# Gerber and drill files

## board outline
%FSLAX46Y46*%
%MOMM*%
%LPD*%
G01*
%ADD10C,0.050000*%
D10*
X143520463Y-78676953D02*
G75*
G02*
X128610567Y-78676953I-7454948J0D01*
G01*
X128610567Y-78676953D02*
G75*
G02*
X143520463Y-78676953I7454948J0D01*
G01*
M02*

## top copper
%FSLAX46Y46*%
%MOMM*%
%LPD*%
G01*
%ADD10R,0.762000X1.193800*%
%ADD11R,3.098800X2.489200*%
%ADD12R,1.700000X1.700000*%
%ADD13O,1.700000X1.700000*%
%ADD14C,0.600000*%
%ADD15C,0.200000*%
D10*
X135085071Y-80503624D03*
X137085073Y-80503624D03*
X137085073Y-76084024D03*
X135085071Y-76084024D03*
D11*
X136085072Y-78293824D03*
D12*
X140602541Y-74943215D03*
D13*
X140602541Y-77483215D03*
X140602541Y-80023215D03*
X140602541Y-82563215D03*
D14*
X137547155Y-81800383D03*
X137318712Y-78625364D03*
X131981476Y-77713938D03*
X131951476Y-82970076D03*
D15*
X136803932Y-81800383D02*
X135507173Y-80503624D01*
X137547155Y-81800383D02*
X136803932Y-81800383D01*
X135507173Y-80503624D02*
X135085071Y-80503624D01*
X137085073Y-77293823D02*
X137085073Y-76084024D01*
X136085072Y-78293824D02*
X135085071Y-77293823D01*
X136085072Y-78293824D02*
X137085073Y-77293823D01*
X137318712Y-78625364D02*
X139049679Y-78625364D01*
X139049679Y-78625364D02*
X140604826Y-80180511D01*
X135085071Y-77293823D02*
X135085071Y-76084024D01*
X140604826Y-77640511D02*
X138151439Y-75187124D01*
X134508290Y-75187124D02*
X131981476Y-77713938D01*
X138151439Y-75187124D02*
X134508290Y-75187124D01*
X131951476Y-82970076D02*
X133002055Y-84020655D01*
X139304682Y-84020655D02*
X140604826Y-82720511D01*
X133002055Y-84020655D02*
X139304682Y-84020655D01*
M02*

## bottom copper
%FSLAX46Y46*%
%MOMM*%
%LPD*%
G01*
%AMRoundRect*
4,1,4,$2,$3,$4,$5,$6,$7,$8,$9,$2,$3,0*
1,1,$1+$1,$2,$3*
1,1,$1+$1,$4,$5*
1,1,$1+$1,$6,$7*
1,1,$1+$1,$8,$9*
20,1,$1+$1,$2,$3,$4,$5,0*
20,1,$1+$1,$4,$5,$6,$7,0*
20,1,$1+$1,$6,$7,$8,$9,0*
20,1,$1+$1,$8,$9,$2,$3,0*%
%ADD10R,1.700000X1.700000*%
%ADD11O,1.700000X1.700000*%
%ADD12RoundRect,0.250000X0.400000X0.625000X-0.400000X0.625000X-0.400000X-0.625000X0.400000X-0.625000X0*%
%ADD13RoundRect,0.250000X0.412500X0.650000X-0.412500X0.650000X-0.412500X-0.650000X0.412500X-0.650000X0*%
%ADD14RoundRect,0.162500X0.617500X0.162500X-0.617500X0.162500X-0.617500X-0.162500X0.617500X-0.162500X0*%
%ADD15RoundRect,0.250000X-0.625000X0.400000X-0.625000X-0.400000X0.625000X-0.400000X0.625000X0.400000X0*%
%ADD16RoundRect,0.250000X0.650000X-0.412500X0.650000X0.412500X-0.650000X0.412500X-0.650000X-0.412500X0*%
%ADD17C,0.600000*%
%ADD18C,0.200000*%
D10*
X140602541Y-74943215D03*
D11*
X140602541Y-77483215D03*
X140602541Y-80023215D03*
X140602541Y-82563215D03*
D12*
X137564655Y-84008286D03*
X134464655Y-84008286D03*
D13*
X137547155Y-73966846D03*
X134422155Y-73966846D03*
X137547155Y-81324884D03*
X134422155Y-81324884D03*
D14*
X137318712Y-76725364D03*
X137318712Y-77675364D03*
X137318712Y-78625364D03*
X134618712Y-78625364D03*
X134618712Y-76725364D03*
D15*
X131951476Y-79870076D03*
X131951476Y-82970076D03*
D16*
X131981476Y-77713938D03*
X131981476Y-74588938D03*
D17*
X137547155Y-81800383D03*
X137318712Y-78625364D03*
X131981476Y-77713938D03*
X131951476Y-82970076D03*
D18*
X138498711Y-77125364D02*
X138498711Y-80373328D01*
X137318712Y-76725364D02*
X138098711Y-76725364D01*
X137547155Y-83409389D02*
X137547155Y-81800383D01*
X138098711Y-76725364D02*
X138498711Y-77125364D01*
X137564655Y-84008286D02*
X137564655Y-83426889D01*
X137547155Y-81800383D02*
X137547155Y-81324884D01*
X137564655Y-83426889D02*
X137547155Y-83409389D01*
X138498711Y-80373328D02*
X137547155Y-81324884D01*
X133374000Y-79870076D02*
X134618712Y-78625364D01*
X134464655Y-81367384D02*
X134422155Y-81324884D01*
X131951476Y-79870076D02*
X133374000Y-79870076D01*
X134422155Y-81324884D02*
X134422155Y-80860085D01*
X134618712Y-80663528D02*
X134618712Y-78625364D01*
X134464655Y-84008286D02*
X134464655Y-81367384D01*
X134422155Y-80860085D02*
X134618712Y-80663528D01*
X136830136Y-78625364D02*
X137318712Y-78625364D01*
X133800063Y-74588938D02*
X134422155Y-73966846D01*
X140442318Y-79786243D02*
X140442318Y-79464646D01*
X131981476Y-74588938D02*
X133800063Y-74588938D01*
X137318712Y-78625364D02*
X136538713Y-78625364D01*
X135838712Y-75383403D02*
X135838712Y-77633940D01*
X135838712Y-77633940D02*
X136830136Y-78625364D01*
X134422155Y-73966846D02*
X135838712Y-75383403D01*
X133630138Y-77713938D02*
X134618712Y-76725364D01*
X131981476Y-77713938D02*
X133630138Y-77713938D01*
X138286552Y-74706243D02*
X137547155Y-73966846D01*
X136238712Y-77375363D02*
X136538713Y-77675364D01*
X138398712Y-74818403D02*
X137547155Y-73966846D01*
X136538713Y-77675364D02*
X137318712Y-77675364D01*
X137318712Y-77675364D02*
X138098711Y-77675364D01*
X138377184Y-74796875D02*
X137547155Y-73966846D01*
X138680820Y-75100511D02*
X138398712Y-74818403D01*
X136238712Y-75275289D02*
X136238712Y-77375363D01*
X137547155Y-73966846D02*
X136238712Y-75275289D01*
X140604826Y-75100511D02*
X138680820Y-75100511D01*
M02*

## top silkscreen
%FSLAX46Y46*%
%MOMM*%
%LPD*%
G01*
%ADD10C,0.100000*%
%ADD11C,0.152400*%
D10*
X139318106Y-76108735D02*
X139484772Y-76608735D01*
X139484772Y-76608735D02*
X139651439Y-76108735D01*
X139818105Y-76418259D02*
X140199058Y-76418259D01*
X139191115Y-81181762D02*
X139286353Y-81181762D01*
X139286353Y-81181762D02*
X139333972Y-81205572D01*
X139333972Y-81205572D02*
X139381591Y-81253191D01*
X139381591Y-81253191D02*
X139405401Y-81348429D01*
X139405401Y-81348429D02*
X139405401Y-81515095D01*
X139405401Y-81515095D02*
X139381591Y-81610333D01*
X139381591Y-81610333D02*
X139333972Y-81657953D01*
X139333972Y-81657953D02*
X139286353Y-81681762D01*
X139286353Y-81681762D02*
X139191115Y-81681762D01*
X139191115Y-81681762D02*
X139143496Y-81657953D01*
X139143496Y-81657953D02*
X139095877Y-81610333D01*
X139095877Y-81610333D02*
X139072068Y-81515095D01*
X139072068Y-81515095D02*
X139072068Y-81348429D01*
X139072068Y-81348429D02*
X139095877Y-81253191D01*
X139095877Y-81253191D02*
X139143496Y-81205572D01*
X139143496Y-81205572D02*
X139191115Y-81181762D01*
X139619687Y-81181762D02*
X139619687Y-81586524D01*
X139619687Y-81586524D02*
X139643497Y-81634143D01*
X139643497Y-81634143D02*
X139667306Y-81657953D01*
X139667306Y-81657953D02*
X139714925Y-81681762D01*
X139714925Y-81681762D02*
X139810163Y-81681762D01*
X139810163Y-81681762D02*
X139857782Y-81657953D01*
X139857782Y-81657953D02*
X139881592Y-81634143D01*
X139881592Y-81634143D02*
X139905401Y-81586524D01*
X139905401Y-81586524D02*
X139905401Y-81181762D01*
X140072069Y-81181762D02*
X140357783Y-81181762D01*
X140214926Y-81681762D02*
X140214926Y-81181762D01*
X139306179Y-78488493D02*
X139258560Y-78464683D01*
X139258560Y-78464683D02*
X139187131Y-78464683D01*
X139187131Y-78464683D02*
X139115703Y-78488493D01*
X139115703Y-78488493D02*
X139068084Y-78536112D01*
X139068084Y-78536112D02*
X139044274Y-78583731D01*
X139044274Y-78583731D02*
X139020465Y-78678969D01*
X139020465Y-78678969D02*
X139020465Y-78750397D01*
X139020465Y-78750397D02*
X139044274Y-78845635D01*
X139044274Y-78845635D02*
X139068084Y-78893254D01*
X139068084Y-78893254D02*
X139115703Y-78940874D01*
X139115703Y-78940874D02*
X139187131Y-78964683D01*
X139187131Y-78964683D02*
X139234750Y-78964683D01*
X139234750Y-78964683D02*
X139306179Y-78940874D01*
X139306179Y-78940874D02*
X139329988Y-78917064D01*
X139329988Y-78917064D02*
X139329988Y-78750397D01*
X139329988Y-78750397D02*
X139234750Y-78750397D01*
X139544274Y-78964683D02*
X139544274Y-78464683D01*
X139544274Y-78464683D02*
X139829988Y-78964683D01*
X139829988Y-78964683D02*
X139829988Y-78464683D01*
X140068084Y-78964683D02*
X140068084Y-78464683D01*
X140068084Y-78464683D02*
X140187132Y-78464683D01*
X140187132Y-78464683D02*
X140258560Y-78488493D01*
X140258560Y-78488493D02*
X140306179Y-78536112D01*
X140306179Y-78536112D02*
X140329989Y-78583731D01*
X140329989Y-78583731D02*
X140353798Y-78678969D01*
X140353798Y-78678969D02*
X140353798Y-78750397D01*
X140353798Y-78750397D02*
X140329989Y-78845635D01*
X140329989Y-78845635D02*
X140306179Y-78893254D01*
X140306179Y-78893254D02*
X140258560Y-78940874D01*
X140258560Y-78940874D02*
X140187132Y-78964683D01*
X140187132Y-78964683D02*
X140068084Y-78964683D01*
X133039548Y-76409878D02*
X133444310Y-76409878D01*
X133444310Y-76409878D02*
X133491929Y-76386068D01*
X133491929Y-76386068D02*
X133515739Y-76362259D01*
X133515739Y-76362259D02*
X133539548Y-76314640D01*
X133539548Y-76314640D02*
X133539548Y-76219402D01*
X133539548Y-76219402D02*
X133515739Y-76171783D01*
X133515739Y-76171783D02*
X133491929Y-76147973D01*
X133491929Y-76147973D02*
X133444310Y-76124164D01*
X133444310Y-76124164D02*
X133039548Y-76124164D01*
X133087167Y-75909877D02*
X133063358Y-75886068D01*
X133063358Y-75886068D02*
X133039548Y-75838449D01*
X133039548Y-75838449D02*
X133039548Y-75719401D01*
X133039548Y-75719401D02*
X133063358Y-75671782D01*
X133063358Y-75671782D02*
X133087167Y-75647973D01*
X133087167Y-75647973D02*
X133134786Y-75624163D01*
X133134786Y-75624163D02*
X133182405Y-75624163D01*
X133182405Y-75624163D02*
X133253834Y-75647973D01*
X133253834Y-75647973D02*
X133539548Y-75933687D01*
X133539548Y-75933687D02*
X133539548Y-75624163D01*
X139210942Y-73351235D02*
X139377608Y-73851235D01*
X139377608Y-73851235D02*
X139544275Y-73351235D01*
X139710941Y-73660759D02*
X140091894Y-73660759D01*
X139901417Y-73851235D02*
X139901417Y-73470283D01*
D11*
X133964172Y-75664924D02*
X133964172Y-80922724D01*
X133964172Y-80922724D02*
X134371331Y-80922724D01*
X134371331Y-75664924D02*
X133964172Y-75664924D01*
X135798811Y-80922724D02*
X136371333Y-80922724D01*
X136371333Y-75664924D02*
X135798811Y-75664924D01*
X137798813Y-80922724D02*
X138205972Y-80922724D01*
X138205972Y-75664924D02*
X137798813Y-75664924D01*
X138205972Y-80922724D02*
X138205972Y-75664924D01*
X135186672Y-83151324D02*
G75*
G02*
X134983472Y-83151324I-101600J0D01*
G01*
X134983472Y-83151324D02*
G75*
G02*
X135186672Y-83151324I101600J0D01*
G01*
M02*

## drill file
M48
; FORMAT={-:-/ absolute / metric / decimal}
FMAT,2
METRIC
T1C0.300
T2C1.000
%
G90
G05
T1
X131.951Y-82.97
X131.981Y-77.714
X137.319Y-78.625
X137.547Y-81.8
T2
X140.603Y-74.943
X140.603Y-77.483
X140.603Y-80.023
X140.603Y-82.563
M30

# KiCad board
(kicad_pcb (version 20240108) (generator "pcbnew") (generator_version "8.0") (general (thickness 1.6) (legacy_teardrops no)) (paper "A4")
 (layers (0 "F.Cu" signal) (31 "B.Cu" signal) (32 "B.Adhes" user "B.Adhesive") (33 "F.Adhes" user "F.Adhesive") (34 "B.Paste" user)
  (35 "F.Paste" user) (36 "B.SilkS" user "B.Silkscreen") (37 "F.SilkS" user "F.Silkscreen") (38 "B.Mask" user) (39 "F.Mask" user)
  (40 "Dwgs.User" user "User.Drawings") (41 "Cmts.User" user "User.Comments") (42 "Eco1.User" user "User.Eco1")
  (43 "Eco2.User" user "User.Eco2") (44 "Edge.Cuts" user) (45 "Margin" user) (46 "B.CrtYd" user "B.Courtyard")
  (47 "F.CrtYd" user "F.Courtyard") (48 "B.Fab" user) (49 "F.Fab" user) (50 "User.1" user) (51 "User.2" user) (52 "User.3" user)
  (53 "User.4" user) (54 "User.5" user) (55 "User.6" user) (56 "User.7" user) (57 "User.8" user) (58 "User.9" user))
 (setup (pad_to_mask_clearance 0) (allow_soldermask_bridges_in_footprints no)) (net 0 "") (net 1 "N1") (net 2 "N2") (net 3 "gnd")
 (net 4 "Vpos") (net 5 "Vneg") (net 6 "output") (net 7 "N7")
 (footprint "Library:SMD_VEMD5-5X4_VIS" (layer "F.Cu") (at 136.085072 78.293824 90)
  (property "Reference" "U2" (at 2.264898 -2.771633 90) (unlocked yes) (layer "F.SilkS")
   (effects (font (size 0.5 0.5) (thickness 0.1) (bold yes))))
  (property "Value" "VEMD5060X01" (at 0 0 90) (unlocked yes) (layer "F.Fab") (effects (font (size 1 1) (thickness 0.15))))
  (fp_line (start 2.6289 -2.1209) (end -2.6289 -2.1209) (stroke (width 0.1524) (type solid)) (layer "F.SilkS"))
  (fp_line (start -2.6289 -2.1209) (end -2.6289 -1.713741) (stroke (width 0.1524) (type solid)) (layer "F.SilkS"))
  (fp_line (start 2.6289 -1.713741) (end 2.6289 -2.1209) (stroke (width 0.1524) (type solid)) (layer "F.SilkS"))
  (fp_line (start -2.6289 -0.286261) (end -2.6289 0.286261) (stroke (width 0.1524) (type solid)) (layer "F.SilkS"))
  (fp_line (start 2.6289 0.286261) (end 2.6289 -0.286261) (stroke (width 0.1524) (type solid)) (layer "F.SilkS"))
  (fp_line (start -2.6289 1.713741) (end -2.6289 2.1209) (stroke (width 0.1524) (type solid)) (layer "F.SilkS"))
  (fp_line (start 2.6289 2.1209) (end 2.6289 1.713741) (stroke (width 0.1524) (type solid)) (layer "F.SilkS"))
  (fp_line (start -2.6289 2.1209) (end 2.6289 2.1209) (stroke (width 0.1524) (type solid)) (layer "F.SilkS"))
  (fp_circle (center -4.8575 -1) (end -4.7559 -1) (stroke (width 0.1524) (type solid)) (fill none) (layer "F.SilkS"))
  (pad "1" smd rect (at -2.2098 -1.000001 90) (size 1.1938 0.762) (layers "F.Cu" "F.Paste" "F.Mask") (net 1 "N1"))
  (pad "2" smd rect (at -2.2098 1.000001 90) (size 1.1938 0.762) (layers "F.Cu" "F.Paste" "F.Mask") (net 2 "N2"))
  (pad "3" smd rect (at 2.2098 1.000001 90) (size 1.1938 0.762) (layers "F.Cu" "F.Paste" "F.Mask") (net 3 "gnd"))
  (pad "4" smd rect (at 2.2098 -1.000001 90) (size 1.1938 0.762) (layers "F.Cu" "F.Paste" "F.Mask") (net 3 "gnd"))
  (pad "5" smd rect (at 0 0 90) (size 2.4892 3.0988) (layers "F.Cu" "F.Paste" "F.Mask") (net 3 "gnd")))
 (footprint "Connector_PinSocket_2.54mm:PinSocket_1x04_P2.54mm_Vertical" (layer "F.Cu") (at 140.602541 74.943215)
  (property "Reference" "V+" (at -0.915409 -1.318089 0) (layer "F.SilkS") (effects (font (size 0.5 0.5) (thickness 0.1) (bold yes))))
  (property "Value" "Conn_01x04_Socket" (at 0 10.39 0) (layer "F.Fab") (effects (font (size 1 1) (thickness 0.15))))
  (pad "1" thru_hole rect (at 0 0) (size 1.7 1.7) (drill 1) (layers "*.Cu" "*.Mask") (remove_unused_layers no) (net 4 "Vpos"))
  (pad "2" thru_hole oval (at 0 2.54) (size 1.7 1.7) (drill 1) (layers "*.Cu" "*.Mask") (remove_unused_layers no) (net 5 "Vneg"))
  (pad "3" thru_hole oval (at 0 5.08) (size 1.7 1.7) (drill 1) (layers "*.Cu" "*.Mask") (remove_unused_layers no) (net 3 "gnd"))
  (pad "4" thru_hole oval (at 0 7.62) (size 1.7 1.7) (drill 1) (layers "*.Cu" "*.Mask") (remove_unused_layers no) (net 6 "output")))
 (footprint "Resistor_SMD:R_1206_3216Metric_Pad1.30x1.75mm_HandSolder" (layer "B.Cu") (at 136.014655 84.008286 180)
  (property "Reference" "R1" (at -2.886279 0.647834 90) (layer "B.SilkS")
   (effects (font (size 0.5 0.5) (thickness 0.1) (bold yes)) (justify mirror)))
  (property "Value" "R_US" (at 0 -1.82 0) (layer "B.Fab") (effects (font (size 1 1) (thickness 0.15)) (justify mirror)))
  (pad "1" smd roundrect (at -1.55 0 180) (size 1.3 1.75) (layers "B.Cu" "B.Paste" "B.Mask") (roundrect_rratio 0.192308) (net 1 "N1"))
  (pad "2" smd roundrect (at 1.55 0 180) (size 1.3 1.75) (layers "B.Cu" "B.Paste" "B.Mask") (roundrect_rratio 0.192308) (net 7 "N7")))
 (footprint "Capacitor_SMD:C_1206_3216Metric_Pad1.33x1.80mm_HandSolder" (layer "B.Cu") (at 135.984655 73.966846 180)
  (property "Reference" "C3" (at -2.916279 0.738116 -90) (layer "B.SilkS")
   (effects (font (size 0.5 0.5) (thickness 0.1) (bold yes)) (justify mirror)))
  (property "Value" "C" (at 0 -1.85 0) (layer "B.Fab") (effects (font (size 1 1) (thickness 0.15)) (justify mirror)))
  (pad "1" smd roundrect (at -1.5625 0 180) (size 1.325 1.8) (layers "B.Cu" "B.Paste" "B.Mask") (roundrect_rratio 0.188679) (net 4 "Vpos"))
  (pad "2" smd roundrect (at 1.5625 0 180) (size 1.325 1.8) (layers "B.Cu" "B.Paste" "B.Mask") (roundrect_rratio 0.188679) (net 3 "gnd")))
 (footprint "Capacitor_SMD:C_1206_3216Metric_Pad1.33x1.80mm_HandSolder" (layer "B.Cu") (at 135.984655 81.324884 180)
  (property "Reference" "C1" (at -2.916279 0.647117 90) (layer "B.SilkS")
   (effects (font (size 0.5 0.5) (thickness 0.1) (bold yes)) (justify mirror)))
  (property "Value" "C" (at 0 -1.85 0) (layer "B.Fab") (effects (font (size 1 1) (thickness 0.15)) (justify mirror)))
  (pad "1" smd roundrect (at -1.5625 0 180) (size 1.325 1.8) (layers "B.Cu" "B.Paste" "B.Mask") (roundrect_rratio 0.188679) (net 1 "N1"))
  (pad "2" smd roundrect (at 1.5625 0 180) (size 1.325 1.8) (layers "B.Cu" "B.Paste" "B.Mask") (roundrect_rratio 0.188679) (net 7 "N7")))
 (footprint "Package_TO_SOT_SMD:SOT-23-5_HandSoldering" (layer "B.Cu") (at 135.968712 77.675364 180)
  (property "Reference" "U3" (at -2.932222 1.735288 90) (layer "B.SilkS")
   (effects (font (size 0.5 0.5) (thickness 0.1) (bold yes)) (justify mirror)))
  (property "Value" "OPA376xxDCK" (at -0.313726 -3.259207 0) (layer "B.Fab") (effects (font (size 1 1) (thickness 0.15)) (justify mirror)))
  (pad "1" smd roundrect (at -1.35 0.95 180) (size 1.56 0.65) (layers "B.Cu" "B.Paste" "B.Mask") (roundrect_rratio 0.25) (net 1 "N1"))
  (pad "2" smd roundrect (at -1.35 0 180) (size 1.56 0.65) (layers "B.Cu" "B.Paste" "B.Mask") (roundrect_rratio 0.25) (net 4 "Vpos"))
  (pad "3" smd roundrect (at -1.35 -0.95 180) (size 1.56 0.65) (layers "B.Cu" "B.Paste" "B.Mask") (roundrect_rratio 0.25) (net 3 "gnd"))
  (pad "4" smd roundrect (at 1.35 -0.95 180) (size 1.56 0.65) (layers "B.Cu" "B.Paste" "B.Mask") (roundrect_rratio 0.25) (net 7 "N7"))
  (pad "5" smd roundrect (at 1.35 0.95 180) (size 1.56 0.65) (layers "B.Cu" "B.Paste" "B.Mask") (roundrect_rratio 0.25) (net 5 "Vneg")))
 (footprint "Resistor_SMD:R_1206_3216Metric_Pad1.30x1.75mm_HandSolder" (layer "B.Cu") (at 131.951476 81.420076 -90)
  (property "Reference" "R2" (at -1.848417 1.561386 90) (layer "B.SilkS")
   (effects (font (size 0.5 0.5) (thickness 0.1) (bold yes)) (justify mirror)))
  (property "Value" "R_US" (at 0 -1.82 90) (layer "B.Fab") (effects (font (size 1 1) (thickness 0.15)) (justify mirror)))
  (pad "1" smd roundrect (at -1.55 0 270) (size 1.3 1.75) (layers "B.Cu" "B.Paste" "B.Mask") (roundrect_rratio 0.192308) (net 7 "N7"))
  (pad "2" smd roundrect (at 1.55 0 270) (size 1.3 1.75) (layers "B.Cu" "B.Paste" "B.Mask") (roundrect_rratio 0.192308) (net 6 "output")))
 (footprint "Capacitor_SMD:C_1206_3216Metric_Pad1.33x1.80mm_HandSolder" (layer "B.Cu") (at 131.981476 76.151438 90)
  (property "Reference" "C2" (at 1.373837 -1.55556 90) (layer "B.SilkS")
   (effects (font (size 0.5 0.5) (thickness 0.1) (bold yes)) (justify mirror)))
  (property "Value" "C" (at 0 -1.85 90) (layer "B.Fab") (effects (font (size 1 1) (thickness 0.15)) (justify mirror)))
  (pad "1" smd roundrect (at -1.5625 0 90) (size 1.325 1.8) (layers "B.Cu" "B.Paste" "B.Mask") (roundrect_rratio 0.188679) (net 5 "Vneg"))
  (pad "2" smd roundrect (at 1.5625 0 90) (size 1.325 1.8) (layers "B.Cu" "B.Paste" "B.Mask") (roundrect_rratio 0.188679) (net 3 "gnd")))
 (gr_circle (center 136.065515 78.676953) (end 143.520284 78.625362) (stroke (width 0.05) (type default)) (fill none) (layer "Edge.Cuts"))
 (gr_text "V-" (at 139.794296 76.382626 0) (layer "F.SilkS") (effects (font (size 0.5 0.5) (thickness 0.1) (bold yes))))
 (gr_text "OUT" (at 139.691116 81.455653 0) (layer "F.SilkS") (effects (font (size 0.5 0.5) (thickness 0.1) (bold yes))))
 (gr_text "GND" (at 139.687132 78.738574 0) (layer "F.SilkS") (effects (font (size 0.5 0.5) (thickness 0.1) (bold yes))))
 (segment (start 136.803932 81.800383) (end 135.507173 80.503624) (width 0.2) (layer "F.Cu") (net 1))
 (segment (start 137.547155 81.800383) (end 136.803932 81.800383) (width 0.2) (layer "F.Cu") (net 1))
 (segment (start 135.507173 80.503624) (end 135.085071 80.503624) (width 0.2) (layer "F.Cu") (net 1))
 (via (at 137.547155 81.800383) (size 0.6) (drill 0.3) (layers "F.Cu" "B.Cu") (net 1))
 (segment (start 138.498711 77.125364) (end 138.498711 80.373328) (width 0.2) (layer "B.Cu") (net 1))
 (segment (start 137.318712 76.725364) (end 138.098711 76.725364) (width 0.2) (layer "B.Cu") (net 1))
 (segment (start 137.547155 83.409389) (end 137.547155 81.800383) (width 0.2) (layer "B.Cu") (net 1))
 (segment (start 138.098711 76.725364) (end 138.498711 77.125364) (width 0.2) (layer "B.Cu") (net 1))
 (segment (start 137.564655 84.008286) (end 137.564655 83.426889) (width 0.2) (layer "B.Cu") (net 1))
 (segment (start 137.547155 81.800383) (end 137.547155 81.324884) (width 0.2) (layer "B.Cu") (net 1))
 (segment (start 137.564655 83.426889) (end 137.547155 83.409389) (width 0.2) (layer "B.Cu") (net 1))
 (segment (start 138.498711 80.373328) (end 137.547155 81.324884) (width 0.2) (layer "B.Cu") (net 1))
 (segment (start 133.374 79.870076) (end 134.618712 78.625364) (width 0.2) (layer "B.Cu") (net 7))
 (segment (start 134.464655 81.367384) (end 134.422155 81.324884) (width 0.2) (layer "B.Cu") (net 7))
 (segment (start 131.951476 79.870076) (end 133.374 79.870076) (width 0.2) (layer "B.Cu") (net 7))
 (segment (start 134.422155 81.324884) (end 134.422155 80.860085) (width 0.2) (layer "B.Cu") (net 7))
 (segment (start 134.618712 80.663528) (end 134.618712 78.625364) (width 0.2) (layer "B.Cu") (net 7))
 (segment (start 134.464655 84.008286) (end 134.464655 81.367384) (width 0.2) (layer "B.Cu") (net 7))
 (segment (start 134.422155 80.860085) (end 134.618712 80.663528) (width 0.2) (layer "B.Cu") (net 7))
 (segment (start 137.085073 77.293823) (end 137.085073 76.084024) (width 0.2) (layer "F.Cu") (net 3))
 (segment (start 136.085072 78.293824) (end 135.085071 77.293823) (width 0.2) (layer "F.Cu") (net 3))
 (segment (start 136.085072 78.293824) (end 137.085073 77.293823) (width 0.2) (layer "F.Cu") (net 3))
 (segment (start 137.318712 78.625364) (end 139.049679 78.625364) (width 0.2) (layer "F.Cu") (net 3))
 (segment (start 139.049679 78.625364) (end 140.604826 80.180511) (width 0.2) (layer "F.Cu") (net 3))
 (segment (start 135.085071 77.293823) (end 135.085071 76.084024) (width 0.2) (layer "F.Cu") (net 3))
 (via (at 137.318712 78.625364) (size 0.6) (drill 0.3) (layers "F.Cu" "B.Cu") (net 3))
 (segment (start 136.830136 78.625364) (end 137.318712 78.625364) (width 0.2) (layer "B.Cu") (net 3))
 (segment (start 133.800063 74.588938) (end 134.422155 73.966846) (width 0.2) (layer "B.Cu") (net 3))
 (segment (start 140.442318 79.786243) (end 140.442318 79.464646) (width 0.2) (layer "B.Cu") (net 3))
 (segment (start 131.981476 74.588938) (end 133.800063 74.588938) (width 0.2) (layer "B.Cu") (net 3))
 (segment (start 137.318712 78.625364) (end 136.538713 78.625364) (width 0.2) (layer "B.Cu") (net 3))
 (segment (start 135.838712 75.383403) (end 135.838712 77.63394) (width 0.2) (layer "B.Cu") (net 3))
 (segment (start 135.838712 77.63394) (end 136.830136 78.625364) (width 0.2) (layer "B.Cu") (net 3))
 (segment (start 134.422155 73.966846) (end 135.838712 75.383403) (width 0.2) (layer "B.Cu") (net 3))
 (segment (start 140.604826 77.640511) (end 138.151439 75.187124) (width 0.2) (layer "F.Cu") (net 5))
 (segment (start 134.50829 75.187124) (end 131.981476 77.713938) (width 0.2) (layer "F.Cu") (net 5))
 (segment (start 138.151439 75.187124) (end 134.50829 75.187124) (width 0.2) (layer "F.Cu") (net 5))
 (via (at 131.981476 77.713938) (size 0.6) (drill 0.3) (layers "F.Cu" "B.Cu") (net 5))
 (segment (start 133.630138 77.713938) (end 134.618712 76.725364) (width 0.2) (layer "B.Cu") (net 5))
 (segment (start 131.981476 77.713938) (end 133.630138 77.713938) (width 0.2) (layer "B.Cu") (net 5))
 (segment (start 138.286552 74.706243) (end 137.547155 73.966846) (width 0.2) (layer "B.Cu") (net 4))
 (segment (start 136.238712 77.375363) (end 136.538713 77.675364) (width 0.2) (layer "B.Cu") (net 4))
 (segment (start 138.398712 74.818403) (end 137.547155 73.966846) (width 0.2) (layer "B.Cu") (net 4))
 (segment (start 136.538713 77.675364) (end 137.318712 77.675364) (width 0.2) (layer "B.Cu") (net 4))
 (segment (start 137.318712 77.675364) (end 138.098711 77.675364) (width 0.2) (layer "B.Cu") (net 4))
 (segment (start 138.377184 74.796875) (end 137.547155 73.966846) (width 0.2) (layer "B.Cu") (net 4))
 (segment (start 138.68082 75.100511) (end 138.398712 74.818403) (width 0.2) (layer "B.Cu") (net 4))
 (segment (start 136.238712 75.275289) (end 136.238712 77.375363) (width 0.2) (layer "B.Cu") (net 4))
 (segment (start 137.547155 73.966846) (end 136.238712 75.275289) (width 0.2) (layer "B.Cu") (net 4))
 (segment (start 140.604826 75.100511) (end 138.68082 75.100511) (width 0.2) (layer "B.Cu") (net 4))
 (segment (start 131.951476 82.970076) (end 133.002055 84.020655) (width 0.2) (layer "F.Cu") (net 6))
 (segment (start 139.304682 84.020655) (end 140.604826 82.720511) (width 0.2) (layer "F.Cu") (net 6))
 (segment (start 133.002055 84.020655) (end 139.304682 84.020655) (width 0.2) (layer "F.Cu") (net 6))
 (via (at 131.951476 82.970076) (size 0.6) (drill 0.3) (layers "F.Cu" "B.Cu") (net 6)))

